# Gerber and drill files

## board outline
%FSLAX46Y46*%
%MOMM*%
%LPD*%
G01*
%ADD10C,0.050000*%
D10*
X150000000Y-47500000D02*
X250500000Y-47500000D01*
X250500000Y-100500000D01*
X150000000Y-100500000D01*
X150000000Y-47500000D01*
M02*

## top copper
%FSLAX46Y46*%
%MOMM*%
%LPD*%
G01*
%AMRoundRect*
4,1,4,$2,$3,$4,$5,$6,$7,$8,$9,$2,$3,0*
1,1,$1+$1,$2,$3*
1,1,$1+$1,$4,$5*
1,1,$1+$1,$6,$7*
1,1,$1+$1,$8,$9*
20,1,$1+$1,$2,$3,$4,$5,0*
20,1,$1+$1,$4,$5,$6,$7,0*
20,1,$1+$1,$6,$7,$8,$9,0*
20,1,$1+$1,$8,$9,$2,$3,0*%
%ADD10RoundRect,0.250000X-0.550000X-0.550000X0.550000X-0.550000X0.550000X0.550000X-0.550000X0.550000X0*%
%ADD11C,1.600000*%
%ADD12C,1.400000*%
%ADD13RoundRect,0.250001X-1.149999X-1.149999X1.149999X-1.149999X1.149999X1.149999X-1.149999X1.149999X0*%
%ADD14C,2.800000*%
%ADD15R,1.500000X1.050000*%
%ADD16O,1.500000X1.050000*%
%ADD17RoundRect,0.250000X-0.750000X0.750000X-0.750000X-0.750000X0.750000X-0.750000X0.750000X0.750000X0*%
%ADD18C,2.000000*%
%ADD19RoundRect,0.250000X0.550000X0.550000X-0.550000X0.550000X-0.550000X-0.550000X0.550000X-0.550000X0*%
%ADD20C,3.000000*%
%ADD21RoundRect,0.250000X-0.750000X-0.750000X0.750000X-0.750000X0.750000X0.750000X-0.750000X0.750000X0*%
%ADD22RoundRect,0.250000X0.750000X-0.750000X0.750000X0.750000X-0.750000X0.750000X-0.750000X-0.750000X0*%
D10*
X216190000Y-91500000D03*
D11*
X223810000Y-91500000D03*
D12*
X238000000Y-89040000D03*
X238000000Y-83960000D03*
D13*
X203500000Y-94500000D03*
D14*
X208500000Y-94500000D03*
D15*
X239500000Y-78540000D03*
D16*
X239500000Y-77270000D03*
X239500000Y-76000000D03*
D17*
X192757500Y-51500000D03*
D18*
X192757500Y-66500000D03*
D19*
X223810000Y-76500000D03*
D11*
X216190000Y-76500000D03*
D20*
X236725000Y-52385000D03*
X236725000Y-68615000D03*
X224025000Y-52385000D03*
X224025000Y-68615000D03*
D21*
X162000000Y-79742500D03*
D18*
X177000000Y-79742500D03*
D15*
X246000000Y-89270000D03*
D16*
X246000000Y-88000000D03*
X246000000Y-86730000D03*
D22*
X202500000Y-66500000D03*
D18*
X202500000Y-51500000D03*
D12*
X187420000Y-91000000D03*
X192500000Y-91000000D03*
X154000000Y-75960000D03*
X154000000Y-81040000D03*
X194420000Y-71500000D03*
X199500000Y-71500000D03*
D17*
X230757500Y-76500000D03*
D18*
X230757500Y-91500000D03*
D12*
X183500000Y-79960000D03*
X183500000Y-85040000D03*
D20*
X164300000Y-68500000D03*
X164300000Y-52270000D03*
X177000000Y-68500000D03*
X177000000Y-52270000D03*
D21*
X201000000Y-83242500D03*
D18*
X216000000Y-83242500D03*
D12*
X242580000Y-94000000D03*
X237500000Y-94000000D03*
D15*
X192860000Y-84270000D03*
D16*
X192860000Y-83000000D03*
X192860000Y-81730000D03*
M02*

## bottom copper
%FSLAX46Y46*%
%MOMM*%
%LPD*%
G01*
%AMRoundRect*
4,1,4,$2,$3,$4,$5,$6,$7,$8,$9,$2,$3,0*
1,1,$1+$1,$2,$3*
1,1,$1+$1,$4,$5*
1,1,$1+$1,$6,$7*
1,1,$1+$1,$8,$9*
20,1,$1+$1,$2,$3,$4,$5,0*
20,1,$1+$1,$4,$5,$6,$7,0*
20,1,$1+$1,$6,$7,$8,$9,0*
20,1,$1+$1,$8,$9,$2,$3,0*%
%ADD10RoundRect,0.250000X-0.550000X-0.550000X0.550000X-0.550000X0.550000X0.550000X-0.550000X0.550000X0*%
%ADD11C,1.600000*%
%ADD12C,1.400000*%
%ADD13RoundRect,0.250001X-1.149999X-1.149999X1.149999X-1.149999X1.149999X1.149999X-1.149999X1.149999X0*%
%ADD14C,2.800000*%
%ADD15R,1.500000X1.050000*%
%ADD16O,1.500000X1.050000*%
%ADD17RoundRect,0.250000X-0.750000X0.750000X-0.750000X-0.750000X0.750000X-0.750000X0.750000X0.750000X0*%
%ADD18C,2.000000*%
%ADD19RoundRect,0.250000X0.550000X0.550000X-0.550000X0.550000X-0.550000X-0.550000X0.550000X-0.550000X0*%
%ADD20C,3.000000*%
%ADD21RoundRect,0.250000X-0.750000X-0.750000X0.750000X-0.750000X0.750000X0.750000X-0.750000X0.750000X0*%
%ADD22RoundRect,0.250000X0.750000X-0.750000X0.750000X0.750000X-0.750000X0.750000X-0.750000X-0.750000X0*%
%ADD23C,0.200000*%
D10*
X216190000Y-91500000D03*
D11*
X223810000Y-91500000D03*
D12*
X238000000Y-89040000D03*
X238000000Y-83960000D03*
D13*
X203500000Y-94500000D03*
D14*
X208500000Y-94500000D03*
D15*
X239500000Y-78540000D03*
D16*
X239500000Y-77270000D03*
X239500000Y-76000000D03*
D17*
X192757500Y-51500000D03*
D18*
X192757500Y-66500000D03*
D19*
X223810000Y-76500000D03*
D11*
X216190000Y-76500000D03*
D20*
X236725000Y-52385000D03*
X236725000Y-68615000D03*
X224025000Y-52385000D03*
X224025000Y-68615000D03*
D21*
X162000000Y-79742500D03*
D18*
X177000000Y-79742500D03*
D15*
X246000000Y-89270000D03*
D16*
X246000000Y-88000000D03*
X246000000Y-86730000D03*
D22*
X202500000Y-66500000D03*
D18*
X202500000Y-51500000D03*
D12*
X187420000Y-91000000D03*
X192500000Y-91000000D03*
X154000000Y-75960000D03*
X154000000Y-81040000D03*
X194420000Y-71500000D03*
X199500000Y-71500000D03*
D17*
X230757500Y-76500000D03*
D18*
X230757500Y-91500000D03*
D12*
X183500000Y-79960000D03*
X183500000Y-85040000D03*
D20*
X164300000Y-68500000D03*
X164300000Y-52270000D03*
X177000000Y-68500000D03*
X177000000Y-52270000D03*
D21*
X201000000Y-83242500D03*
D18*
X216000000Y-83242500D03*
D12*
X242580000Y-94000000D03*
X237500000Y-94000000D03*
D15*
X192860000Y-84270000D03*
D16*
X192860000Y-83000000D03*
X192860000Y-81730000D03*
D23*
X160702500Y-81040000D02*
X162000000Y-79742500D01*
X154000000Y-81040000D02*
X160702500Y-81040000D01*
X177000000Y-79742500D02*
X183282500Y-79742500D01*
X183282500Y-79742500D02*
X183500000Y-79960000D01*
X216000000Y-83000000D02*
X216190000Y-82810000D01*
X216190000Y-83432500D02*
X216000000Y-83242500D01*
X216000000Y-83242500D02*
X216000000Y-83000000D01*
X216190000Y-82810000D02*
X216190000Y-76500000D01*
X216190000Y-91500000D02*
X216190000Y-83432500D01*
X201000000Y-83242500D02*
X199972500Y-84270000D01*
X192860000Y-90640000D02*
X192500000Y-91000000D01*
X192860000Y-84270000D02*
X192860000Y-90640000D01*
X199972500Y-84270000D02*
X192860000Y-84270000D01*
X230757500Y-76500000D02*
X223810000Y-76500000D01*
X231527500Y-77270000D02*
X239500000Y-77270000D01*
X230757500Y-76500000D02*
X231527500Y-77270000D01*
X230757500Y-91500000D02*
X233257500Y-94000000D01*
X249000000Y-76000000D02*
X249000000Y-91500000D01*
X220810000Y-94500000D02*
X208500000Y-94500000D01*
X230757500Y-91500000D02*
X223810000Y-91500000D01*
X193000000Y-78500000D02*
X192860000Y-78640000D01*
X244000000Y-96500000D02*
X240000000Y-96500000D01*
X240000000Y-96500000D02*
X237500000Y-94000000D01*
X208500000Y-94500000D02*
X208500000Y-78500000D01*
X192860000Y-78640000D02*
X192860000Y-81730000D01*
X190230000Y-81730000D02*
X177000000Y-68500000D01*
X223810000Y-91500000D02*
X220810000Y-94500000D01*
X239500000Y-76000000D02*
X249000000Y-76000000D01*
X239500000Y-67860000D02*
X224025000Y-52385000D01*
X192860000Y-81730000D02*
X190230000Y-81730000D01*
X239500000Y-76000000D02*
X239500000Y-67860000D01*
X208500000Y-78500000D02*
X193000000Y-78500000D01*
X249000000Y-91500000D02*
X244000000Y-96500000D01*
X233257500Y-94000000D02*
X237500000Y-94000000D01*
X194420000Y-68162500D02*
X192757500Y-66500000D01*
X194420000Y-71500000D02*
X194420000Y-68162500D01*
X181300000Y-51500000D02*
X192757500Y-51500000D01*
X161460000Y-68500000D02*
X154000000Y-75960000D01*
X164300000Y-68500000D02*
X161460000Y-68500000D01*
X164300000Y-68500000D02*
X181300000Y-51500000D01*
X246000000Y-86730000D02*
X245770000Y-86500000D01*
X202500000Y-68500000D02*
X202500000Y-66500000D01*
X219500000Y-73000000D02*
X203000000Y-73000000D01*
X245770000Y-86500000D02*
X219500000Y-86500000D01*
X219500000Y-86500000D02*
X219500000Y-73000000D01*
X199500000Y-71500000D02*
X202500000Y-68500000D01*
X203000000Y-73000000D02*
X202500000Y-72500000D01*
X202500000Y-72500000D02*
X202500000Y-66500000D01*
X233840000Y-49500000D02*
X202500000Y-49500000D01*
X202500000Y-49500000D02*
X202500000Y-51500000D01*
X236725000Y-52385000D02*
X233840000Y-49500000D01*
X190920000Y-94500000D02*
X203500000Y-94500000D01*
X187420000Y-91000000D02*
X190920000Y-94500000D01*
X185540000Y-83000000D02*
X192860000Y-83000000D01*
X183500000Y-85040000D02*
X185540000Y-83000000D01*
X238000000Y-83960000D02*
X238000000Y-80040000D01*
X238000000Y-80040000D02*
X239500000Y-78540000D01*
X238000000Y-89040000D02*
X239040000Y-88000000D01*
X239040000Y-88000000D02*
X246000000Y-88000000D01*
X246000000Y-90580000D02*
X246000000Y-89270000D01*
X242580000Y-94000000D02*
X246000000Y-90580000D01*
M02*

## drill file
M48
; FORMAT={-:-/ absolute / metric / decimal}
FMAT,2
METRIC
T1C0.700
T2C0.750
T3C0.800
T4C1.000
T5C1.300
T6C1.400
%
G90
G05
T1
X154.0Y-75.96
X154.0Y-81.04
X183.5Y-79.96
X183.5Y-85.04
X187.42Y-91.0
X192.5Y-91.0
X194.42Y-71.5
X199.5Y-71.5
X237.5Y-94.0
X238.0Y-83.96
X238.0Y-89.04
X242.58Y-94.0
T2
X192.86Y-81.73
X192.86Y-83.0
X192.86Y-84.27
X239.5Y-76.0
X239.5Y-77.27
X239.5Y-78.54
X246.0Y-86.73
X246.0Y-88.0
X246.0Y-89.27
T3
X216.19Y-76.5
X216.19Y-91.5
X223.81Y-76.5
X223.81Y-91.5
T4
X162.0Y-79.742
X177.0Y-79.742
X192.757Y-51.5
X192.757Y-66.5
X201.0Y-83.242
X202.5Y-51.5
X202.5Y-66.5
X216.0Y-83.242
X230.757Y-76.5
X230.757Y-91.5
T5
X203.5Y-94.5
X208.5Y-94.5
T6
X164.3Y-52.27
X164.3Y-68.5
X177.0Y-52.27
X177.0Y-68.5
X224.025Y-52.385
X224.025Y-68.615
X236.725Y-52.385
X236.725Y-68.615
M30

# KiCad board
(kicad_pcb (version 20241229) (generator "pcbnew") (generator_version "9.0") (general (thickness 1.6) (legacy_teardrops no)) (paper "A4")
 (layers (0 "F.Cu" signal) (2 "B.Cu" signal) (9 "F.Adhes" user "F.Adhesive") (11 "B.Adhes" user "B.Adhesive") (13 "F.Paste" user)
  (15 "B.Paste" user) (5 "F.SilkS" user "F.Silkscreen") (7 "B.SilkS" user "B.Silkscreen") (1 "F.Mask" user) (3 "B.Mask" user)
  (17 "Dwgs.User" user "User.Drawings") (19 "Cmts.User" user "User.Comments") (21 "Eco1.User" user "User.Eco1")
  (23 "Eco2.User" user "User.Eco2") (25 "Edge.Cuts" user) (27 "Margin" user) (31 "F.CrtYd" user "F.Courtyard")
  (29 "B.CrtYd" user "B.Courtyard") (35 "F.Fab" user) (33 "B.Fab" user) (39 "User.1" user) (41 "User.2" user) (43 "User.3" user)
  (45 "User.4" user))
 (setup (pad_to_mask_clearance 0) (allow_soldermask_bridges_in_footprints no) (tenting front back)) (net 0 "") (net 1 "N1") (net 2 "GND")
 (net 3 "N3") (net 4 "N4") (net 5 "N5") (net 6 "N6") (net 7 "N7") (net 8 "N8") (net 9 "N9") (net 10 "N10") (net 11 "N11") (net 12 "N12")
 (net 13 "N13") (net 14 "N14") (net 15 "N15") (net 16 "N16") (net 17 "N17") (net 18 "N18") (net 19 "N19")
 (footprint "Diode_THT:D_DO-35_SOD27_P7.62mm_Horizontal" (layer "F.Cu") (at 216.19 91.5)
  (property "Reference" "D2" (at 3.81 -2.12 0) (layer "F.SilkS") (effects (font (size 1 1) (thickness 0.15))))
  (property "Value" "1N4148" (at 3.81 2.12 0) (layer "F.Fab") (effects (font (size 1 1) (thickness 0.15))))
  (pad "1" thru_hole roundrect (at 0 0) (size 1.6 1.6) (drill 0.8) (layers "*.Cu" "*.Mask") (remove_unused_layers no)
   (roundrect_rratio 0.15625) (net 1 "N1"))
  (pad "2" thru_hole circle (at 7.62 0) (size 1.6 1.6) (drill 0.8) (layers "*.Cu" "*.Mask") (remove_unused_layers no) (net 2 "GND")))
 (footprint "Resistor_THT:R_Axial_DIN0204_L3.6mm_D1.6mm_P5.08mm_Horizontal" (layer "F.Cu") (at 238 89.04 90)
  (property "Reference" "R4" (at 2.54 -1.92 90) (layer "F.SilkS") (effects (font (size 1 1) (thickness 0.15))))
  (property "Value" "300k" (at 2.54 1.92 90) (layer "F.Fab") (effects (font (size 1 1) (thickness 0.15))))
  (pad "1" thru_hole circle (at 0 0 90) (size 1.4 1.4) (drill 0.7) (layers "*.Cu" "*.Mask") (remove_unused_layers no) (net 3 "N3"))
  (pad "2" thru_hole circle (at 5.08 0 90) (size 1.4 1.4) (drill 0.7) (layers "*.Cu" "*.Mask") (remove_unused_layers no) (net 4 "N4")))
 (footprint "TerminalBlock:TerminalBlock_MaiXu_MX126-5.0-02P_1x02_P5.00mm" (layer "F.Cu") (at 203.5 94.5)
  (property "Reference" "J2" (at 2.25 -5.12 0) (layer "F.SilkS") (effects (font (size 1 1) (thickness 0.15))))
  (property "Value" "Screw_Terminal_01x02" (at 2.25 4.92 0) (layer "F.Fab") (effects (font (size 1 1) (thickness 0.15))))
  (pad "1" thru_hole roundrect (at 0 0) (size 2.8 2.8) (drill 1.3) (layers "*.Cu" "*.Mask") (remove_unused_layers no)
   (roundrect_rratio 0.089286) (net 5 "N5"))
  (pad "2" thru_hole circle (at 5 0) (size 2.8 2.8) (drill 1.3) (layers "*.Cu" "*.Mask") (remove_unused_layers no) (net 2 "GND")))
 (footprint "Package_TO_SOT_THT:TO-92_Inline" (layer "F.Cu") (at 239.5 78.54 90)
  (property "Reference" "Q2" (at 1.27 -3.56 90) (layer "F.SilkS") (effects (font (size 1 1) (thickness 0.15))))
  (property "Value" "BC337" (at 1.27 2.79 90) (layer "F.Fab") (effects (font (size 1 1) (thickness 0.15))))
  (pad "1" thru_hole rect (at 0 0 90) (size 1.05 1.5) (drill 0.75) (layers "*.Cu" "*.Mask") (remove_unused_layers no) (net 4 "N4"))
  (pad "2" thru_hole oval (at 1.27 0 90) (size 1.05 1.5) (drill 0.75) (layers "*.Cu" "*.Mask") (remove_unused_layers no) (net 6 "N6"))
  (pad "3" thru_hole oval (at 2.54 0 90) (size 1.05 1.5) (drill 0.75) (layers "*.Cu" "*.Mask") (remove_unused_layers no) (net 2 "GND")))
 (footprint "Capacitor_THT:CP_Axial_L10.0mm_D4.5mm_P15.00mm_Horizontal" (layer "F.Cu") (at 192.7575 51.5 -90)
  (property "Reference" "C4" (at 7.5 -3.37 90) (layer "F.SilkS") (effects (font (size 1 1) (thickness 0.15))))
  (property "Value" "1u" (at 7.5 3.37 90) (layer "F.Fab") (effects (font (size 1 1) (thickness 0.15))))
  (pad "1" thru_hole roundrect (at 0 0 270) (size 2 2) (drill 1) (layers "*.Cu" "*.Mask") (remove_unused_layers no) (roundrect_rratio 0.125)
   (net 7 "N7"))
  (pad "2" thru_hole circle (at 15 0 270) (size 2 2) (drill 1) (layers "*.Cu" "*.Mask") (remove_unused_layers no) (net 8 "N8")))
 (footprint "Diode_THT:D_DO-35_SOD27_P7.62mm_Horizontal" (layer "F.Cu") (at 223.81 76.5 180)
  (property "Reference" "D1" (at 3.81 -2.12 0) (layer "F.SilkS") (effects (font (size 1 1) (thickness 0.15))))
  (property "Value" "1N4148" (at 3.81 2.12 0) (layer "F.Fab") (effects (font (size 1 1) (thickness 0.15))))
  (pad "1" thru_hole roundrect (at 0 0 180) (size 1.6 1.6) (drill 0.8) (layers "*.Cu" "*.Mask") (remove_unused_layers no)
   (roundrect_rratio 0.15625) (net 6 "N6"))
  (pad "2" thru_hole circle (at 7.62 0 180) (size 1.6 1.6) (drill 0.8) (layers "*.Cu" "*.Mask") (remove_unused_layers no) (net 1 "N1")))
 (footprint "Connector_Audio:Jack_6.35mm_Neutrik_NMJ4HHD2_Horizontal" (layer "F.Cu") (at 224.025 52.385)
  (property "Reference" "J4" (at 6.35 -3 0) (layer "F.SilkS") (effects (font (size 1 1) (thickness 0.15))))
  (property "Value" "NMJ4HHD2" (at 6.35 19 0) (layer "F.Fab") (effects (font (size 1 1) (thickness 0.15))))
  (pad "S" thru_hole circle (at 12.7 0) (size 3 3) (drill 1.4) (layers "*.Cu" "*.Mask") (remove_unused_layers no) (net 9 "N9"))
  (pad "SN" thru_hole circle (at 12.7 16.23) (size 3 3) (drill 1.4) (layers "*.Cu" "*.Mask") (remove_unused_layers no) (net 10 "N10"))
  (pad "T" thru_hole circle (at 0 0) (size 3 3) (drill 1.4) (layers "*.Cu" "*.Mask") (remove_unused_layers no) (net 2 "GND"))
  (pad "TN" thru_hole circle (at 0 16.23) (size 3 3) (drill 1.4) (layers "*.Cu" "*.Mask") (remove_unused_layers no) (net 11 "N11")))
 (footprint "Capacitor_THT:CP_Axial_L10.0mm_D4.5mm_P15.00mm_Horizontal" (layer "F.Cu") (at 162 79.7425)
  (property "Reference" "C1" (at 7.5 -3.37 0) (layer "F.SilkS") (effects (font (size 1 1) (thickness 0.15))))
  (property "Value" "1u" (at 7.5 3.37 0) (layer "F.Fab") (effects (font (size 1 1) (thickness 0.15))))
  (pad "1" thru_hole roundrect (at 0 0) (size 2 2) (drill 1) (layers "*.Cu" "*.Mask") (remove_unused_layers no) (roundrect_rratio 0.125)
   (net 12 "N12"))
  (pad "2" thru_hole circle (at 15 0) (size 2 2) (drill 1) (layers "*.Cu" "*.Mask") (remove_unused_layers no) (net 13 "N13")))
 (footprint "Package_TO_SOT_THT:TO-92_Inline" (layer "F.Cu") (at 246 89.27 90)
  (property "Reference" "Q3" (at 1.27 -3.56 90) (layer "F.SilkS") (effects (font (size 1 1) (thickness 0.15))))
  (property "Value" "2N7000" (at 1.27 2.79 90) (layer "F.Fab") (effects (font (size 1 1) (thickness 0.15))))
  (pad "1" thru_hole rect (at 0 0 90) (size 1.05 1.5) (drill 0.75) (layers "*.Cu" "*.Mask") (remove_unused_layers no) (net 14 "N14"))
  (pad "2" thru_hole oval (at 1.27 0 90) (size 1.05 1.5) (drill 0.75) (layers "*.Cu" "*.Mask") (remove_unused_layers no) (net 3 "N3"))
  (pad "3" thru_hole oval (at 2.54 0 90) (size 1.05 1.5) (drill 0.75) (layers "*.Cu" "*.Mask") (remove_unused_layers no) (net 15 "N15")))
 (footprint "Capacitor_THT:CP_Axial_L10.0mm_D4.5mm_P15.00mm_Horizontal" (layer "F.Cu") (at 202.5 66.5 90)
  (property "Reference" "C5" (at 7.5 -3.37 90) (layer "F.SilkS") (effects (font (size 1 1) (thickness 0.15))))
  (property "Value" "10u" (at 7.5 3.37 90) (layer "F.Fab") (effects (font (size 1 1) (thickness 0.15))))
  (pad "1" thru_hole roundrect (at 0 0 90) (size 2 2) (drill 1) (layers "*.Cu" "*.Mask") (remove_unused_layers no) (roundrect_rratio 0.125)
   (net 15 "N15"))
  (pad "2" thru_hole circle (at 15 0 90) (size 2 2) (drill 1) (layers "*.Cu" "*.Mask") (remove_unused_layers no) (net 9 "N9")))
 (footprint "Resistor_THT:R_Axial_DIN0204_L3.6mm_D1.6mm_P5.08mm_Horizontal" (layer "F.Cu") (at 187.42 91)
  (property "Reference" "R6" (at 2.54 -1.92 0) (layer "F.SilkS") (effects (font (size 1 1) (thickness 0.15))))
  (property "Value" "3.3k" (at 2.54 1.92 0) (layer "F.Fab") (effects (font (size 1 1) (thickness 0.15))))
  (pad "1" thru_hole circle (at 0 0) (size 1.4 1.4) (drill 0.7) (layers "*.Cu" "*.Mask") (remove_unused_layers no) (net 5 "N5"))
  (pad "2" thru_hole circle (at 5.08 0) (size 1.4 1.4) (drill 0.7) (layers "*.Cu" "*.Mask") (remove_unused_layers no) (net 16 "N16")))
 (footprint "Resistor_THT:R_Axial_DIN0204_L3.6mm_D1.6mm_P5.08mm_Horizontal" (layer "F.Cu") (at 154 75.96 -90)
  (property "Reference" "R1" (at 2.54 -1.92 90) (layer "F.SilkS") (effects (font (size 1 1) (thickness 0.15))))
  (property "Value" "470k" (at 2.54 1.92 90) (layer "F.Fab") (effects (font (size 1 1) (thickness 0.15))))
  (pad "1" thru_hole circle (at 0 0 270) (size 1.4 1.4) (drill 0.7) (layers "*.Cu" "*.Mask") (remove_unused_layers no) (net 7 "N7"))
  (pad "2" thru_hole circle (at 5.08 0 270) (size 1.4 1.4) (drill 0.7) (layers "*.Cu" "*.Mask") (remove_unused_layers no) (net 12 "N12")))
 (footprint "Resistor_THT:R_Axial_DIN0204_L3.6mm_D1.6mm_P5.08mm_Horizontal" (layer "F.Cu") (at 194.42 71.5)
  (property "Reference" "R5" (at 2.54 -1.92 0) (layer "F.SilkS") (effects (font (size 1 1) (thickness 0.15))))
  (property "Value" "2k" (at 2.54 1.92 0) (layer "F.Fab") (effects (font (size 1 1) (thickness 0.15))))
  (pad "1" thru_hole circle (at 0 0) (size 1.4 1.4) (drill 0.7) (layers "*.Cu" "*.Mask") (remove_unused_layers no) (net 8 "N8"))
  (pad "2" thru_hole circle (at 5.08 0) (size 1.4 1.4) (drill 0.7) (layers "*.Cu" "*.Mask") (remove_unused_layers no) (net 15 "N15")))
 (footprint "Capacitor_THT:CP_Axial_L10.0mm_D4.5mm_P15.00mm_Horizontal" (layer "F.Cu") (at 230.7575 76.5 -90)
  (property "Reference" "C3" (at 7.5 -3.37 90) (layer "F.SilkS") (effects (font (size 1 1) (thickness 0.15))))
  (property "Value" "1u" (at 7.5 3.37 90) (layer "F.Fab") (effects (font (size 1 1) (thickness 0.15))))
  (pad "1" thru_hole roundrect (at 0 0 270) (size 2 2) (drill 1) (layers "*.Cu" "*.Mask") (remove_unused_layers no) (roundrect_rratio 0.125)
   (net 6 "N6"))
  (pad "2" thru_hole circle (at 15 0 270) (size 2 2) (drill 1) (layers "*.Cu" "*.Mask") (remove_unused_layers no) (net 2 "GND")))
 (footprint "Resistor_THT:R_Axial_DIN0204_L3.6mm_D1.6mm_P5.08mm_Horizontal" (layer "F.Cu") (at 183.5 79.96 -90)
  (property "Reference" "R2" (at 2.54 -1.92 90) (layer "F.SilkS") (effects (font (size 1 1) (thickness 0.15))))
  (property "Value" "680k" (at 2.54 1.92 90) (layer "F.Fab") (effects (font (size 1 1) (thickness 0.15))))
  (pad "1" thru_hole circle (at 0 0 270) (size 1.4 1.4) (drill 0.7) (layers "*.Cu" "*.Mask") (remove_unused_layers no) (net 13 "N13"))
  (pad "2" thru_hole circle (at 5.08 0 270) (size 1.4 1.4) (drill 0.7) (layers "*.Cu" "*.Mask") (remove_unused_layers no) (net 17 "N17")))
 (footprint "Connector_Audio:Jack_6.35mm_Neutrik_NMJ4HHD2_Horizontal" (layer "F.Cu") (at 177 68.5 180)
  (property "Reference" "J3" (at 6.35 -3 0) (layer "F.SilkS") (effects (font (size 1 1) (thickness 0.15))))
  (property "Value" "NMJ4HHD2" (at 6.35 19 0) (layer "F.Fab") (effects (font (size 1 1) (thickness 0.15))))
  (pad "S" thru_hole circle (at 12.7 0 180) (size 3 3) (drill 1.4) (layers "*.Cu" "*.Mask") (remove_unused_layers no) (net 7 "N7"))
  (pad "SN" thru_hole circle (at 12.7 16.23 180) (size 3 3) (drill 1.4) (layers "*.Cu" "*.Mask") (remove_unused_layers no) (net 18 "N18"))
  (pad "T" thru_hole circle (at 0 0 180) (size 3 3) (drill 1.4) (layers "*.Cu" "*.Mask") (remove_unused_layers no) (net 2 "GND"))
  (pad "TN" thru_hole circle (at 0 16.23 180) (size 3 3) (drill 1.4) (layers "*.Cu" "*.Mask") (remove_unused_layers no) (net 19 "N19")))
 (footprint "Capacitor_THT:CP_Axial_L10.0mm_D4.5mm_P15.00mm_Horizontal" (layer "F.Cu") (at 201 83.2425)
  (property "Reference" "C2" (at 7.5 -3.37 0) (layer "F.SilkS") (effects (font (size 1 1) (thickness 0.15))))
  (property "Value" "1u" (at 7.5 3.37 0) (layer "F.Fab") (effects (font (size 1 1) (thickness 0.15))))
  (pad "1" thru_hole roundrect (at 0 0) (size 2 2) (drill 1) (layers "*.Cu" "*.Mask") (remove_unused_layers no) (roundrect_rratio 0.125)
   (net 16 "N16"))
  (pad "2" thru_hole circle (at 15 0) (size 2 2) (drill 1) (layers "*.Cu" "*.Mask") (remove_unused_layers no) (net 1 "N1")))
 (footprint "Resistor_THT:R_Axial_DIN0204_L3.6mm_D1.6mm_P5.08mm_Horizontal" (layer "F.Cu") (at 242.58 94 180)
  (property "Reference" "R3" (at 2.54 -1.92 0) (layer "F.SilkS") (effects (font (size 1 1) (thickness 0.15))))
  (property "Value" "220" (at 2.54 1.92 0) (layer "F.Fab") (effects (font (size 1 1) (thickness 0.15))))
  (pad "1" thru_hole circle (at 0 0 180) (size 1.4 1.4) (drill 0.7) (layers "*.Cu" "*.Mask") (remove_unused_layers no) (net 14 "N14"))
  (pad "2" thru_hole circle (at 5.08 0 180) (size 1.4 1.4) (drill 0.7) (layers "*.Cu" "*.Mask") (remove_unused_layers no) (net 2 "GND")))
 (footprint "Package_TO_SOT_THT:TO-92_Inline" (layer "F.Cu") (at 192.86 84.27 90)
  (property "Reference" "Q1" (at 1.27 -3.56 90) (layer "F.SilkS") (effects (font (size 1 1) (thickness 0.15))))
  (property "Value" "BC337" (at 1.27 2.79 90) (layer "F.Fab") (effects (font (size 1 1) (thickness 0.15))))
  (pad "1" thru_hole rect (at 0 0 90) (size 1.05 1.5) (drill 0.75) (layers "*.Cu" "*.Mask") (remove_unused_layers no) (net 16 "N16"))
  (pad "2" thru_hole oval (at 1.27 0 90) (size 1.05 1.5) (drill 0.75) (layers "*.Cu" "*.Mask") (remove_unused_layers no) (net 17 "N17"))
  (pad "3" thru_hole oval (at 2.54 0 90) (size 1.05 1.5) (drill 0.75) (layers "*.Cu" "*.Mask") (remove_unused_layers no) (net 2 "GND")))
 (gr_rect (start 150 47.5) (end 250.5 100.5) (stroke (width 0.05) (type default)) (fill no) (layer "Edge.Cuts"))
 (segment (start 160.7025 81.04) (end 162 79.7425) (width 0.2) (layer "B.Cu") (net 12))
 (segment (start 154 81.04) (end 160.7025 81.04) (width 0.2) (layer "B.Cu") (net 12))
 (segment (start 177 79.7425) (end 183.2825 79.7425) (width 0.2) (layer "B.Cu") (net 13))
 (segment (start 183.2825 79.7425) (end 183.5 79.96) (width 0.2) (layer "B.Cu") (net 13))
 (segment (start 216 83) (end 216.19 82.81) (width 0.2) (layer "B.Cu") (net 1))
 (segment (start 216.19 83.4325) (end 216 83.2425) (width 0.2) (layer "B.Cu") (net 1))
 (segment (start 216 83.2425) (end 216 83) (width 0.2) (layer "B.Cu") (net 1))
 (segment (start 216.19 82.81) (end 216.19 76.5) (width 0.2) (layer "B.Cu") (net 1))
 (segment (start 216.19 91.5) (end 216.19 83.4325) (width 0.2) (layer "B.Cu") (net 1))
 (segment (start 201 83.2425) (end 199.9725 84.27) (width 0.2) (layer "B.Cu") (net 16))
 (segment (start 192.86 90.64) (end 192.5 91) (width 0.2) (layer "B.Cu") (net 16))
 (segment (start 192.86 84.27) (end 192.86 90.64) (width 0.2) (layer "B.Cu") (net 16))
 (segment (start 199.9725 84.27) (end 192.86 84.27) (width 0.2) (layer "B.Cu") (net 16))
 (segment (start 230.7575 76.5) (end 223.81 76.5) (width 0.2) (layer "B.Cu") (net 6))
 (segment (start 231.5275 77.27) (end 239.5 77.27) (width 0.2) (layer "B.Cu") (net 6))
 (segment (start 230.7575 76.5) (end 231.5275 77.27) (width 0.2) (layer "B.Cu") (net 6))
 (segment (start 230.7575 91.5) (end 233.2575 94) (width 0.2) (layer "B.Cu") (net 2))
 (segment (start 249 76) (end 249 91.5) (width 0.2) (layer "B.Cu") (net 2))
 (segment (start 220.81 94.5) (end 208.5 94.5) (width 0.2) (layer "B.Cu") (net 2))
 (segment (start 230.7575 91.5) (end 223.81 91.5) (width 0.2) (layer "B.Cu") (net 2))
 (segment (start 193 78.5) (end 192.86 78.64) (width 0.2) (layer "B.Cu") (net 2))
 (segment (start 244 96.5) (end 240 96.5) (width 0.2) (layer "B.Cu") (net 2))
 (segment (start 240 96.5) (end 237.5 94) (width 0.2) (layer "B.Cu") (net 2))
 (segment (start 208.5 94.5) (end 208.5 78.5) (width 0.2) (layer "B.Cu") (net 2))
 (segment (start 192.86 78.64) (end 192.86 81.73) (width 0.2) (layer "B.Cu") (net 2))
 (segment (start 190.23 81.73) (end 177 68.5) (width 0.2) (layer "B.Cu") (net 2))
 (segment (start 223.81 91.5) (end 220.81 94.5) (width 0.2) (layer "B.Cu") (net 2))
 (segment (start 239.5 76) (end 249 76) (width 0.2) (layer "B.Cu") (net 2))
 (segment (start 239.5 67.86) (end 224.025 52.385) (width 0.2) (layer "B.Cu") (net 2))
 (segment (start 192.86 81.73) (end 190.23 81.73) (width 0.2) (layer "B.Cu") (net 2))
 (segment (start 239.5 76) (end 239.5 67.86) (width 0.2) (layer "B.Cu") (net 2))
 (segment (start 208.5 78.5) (end 193 78.5) (width 0.2) (layer "B.Cu") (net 2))
 (segment (start 249 91.5) (end 244 96.5) (width 0.2) (layer "B.Cu") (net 2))
 (segment (start 233.2575 94) (end 237.5 94) (width 0.2) (layer "B.Cu") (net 2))
 (segment (start 194.42 68.1625) (end 192.7575 66.5) (width 0.2) (layer "B.Cu") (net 8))
 (segment (start 194.42 71.5) (end 194.42 68.1625) (width 0.2) (layer "B.Cu") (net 8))
 (segment (start 181.3 51.5) (end 192.7575 51.5) (width 0.2) (layer "B.Cu") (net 7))
 (segment (start 161.46 68.5) (end 154 75.96) (width 0.2) (layer "B.Cu") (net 7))
 (segment (start 164.3 68.5) (end 161.46 68.5) (width 0.2) (layer "B.Cu") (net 7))
 (segment (start 164.3 68.5) (end 181.3 51.5) (width 0.2) (layer "B.Cu") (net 7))
 (segment (start 246 86.73) (end 245.77 86.5) (width 0.2) (layer "B.Cu") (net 15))
 (segment (start 202.5 68.5) (end 202.5 66.5) (width 0.2) (layer "B.Cu") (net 15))
 (segment (start 219.5 73) (end 203 73) (width 0.2) (layer "B.Cu") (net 15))
 (segment (start 245.77 86.5) (end 219.5 86.5) (width 0.2) (layer "B.Cu") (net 15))
 (segment (start 219.5 86.5) (end 219.5 73) (width 0.2) (layer "B.Cu") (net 15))
 (segment (start 199.5 71.5) (end 202.5 68.5) (width 0.2) (layer "B.Cu") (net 15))
 (segment (start 203 73) (end 202.5 72.5) (width 0.2) (layer "B.Cu") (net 15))
 (segment (start 202.5 72.5) (end 202.5 66.5) (width 0.2) (layer "B.Cu") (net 15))
 (segment (start 233.84 49.5) (end 202.5 49.5) (width 0.2) (layer "B.Cu") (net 9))
 (segment (start 202.5 49.5) (end 202.5 51.5) (width 0.2) (layer "B.Cu") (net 9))
 (segment (start 236.725 52.385) (end 233.84 49.5) (width 0.2) (layer "B.Cu") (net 9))
 (segment (start 190.92 94.5) (end 203.5 94.5) (width 0.2) (layer "B.Cu") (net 5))
 (segment (start 187.42 91) (end 190.92 94.5) (width 0.2) (layer "B.Cu") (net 5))
 (segment (start 185.54 83) (end 192.86 83) (width 0.2) (layer "B.Cu") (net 17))
 (segment (start 183.5 85.04) (end 185.54 83) (width 0.2) (layer "B.Cu") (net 17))
 (segment (start 238 83.96) (end 238 80.04) (width 0.2) (layer "B.Cu") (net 4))
 (segment (start 238 80.04) (end 239.5 78.54) (width 0.2) (layer "B.Cu") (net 4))
 (segment (start 238 89.04) (end 239.04 88) (width 0.2) (layer "B.Cu") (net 3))
 (segment (start 239.04 88) (end 246 88) (width 0.2) (layer "B.Cu") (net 3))
 (segment (start 246 90.58) (end 246 89.27) (width 0.2) (layer "B.Cu") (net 14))
 (segment (start 242.58 94) (end 246 90.58) (width 0.2) (layer "B.Cu") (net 14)))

